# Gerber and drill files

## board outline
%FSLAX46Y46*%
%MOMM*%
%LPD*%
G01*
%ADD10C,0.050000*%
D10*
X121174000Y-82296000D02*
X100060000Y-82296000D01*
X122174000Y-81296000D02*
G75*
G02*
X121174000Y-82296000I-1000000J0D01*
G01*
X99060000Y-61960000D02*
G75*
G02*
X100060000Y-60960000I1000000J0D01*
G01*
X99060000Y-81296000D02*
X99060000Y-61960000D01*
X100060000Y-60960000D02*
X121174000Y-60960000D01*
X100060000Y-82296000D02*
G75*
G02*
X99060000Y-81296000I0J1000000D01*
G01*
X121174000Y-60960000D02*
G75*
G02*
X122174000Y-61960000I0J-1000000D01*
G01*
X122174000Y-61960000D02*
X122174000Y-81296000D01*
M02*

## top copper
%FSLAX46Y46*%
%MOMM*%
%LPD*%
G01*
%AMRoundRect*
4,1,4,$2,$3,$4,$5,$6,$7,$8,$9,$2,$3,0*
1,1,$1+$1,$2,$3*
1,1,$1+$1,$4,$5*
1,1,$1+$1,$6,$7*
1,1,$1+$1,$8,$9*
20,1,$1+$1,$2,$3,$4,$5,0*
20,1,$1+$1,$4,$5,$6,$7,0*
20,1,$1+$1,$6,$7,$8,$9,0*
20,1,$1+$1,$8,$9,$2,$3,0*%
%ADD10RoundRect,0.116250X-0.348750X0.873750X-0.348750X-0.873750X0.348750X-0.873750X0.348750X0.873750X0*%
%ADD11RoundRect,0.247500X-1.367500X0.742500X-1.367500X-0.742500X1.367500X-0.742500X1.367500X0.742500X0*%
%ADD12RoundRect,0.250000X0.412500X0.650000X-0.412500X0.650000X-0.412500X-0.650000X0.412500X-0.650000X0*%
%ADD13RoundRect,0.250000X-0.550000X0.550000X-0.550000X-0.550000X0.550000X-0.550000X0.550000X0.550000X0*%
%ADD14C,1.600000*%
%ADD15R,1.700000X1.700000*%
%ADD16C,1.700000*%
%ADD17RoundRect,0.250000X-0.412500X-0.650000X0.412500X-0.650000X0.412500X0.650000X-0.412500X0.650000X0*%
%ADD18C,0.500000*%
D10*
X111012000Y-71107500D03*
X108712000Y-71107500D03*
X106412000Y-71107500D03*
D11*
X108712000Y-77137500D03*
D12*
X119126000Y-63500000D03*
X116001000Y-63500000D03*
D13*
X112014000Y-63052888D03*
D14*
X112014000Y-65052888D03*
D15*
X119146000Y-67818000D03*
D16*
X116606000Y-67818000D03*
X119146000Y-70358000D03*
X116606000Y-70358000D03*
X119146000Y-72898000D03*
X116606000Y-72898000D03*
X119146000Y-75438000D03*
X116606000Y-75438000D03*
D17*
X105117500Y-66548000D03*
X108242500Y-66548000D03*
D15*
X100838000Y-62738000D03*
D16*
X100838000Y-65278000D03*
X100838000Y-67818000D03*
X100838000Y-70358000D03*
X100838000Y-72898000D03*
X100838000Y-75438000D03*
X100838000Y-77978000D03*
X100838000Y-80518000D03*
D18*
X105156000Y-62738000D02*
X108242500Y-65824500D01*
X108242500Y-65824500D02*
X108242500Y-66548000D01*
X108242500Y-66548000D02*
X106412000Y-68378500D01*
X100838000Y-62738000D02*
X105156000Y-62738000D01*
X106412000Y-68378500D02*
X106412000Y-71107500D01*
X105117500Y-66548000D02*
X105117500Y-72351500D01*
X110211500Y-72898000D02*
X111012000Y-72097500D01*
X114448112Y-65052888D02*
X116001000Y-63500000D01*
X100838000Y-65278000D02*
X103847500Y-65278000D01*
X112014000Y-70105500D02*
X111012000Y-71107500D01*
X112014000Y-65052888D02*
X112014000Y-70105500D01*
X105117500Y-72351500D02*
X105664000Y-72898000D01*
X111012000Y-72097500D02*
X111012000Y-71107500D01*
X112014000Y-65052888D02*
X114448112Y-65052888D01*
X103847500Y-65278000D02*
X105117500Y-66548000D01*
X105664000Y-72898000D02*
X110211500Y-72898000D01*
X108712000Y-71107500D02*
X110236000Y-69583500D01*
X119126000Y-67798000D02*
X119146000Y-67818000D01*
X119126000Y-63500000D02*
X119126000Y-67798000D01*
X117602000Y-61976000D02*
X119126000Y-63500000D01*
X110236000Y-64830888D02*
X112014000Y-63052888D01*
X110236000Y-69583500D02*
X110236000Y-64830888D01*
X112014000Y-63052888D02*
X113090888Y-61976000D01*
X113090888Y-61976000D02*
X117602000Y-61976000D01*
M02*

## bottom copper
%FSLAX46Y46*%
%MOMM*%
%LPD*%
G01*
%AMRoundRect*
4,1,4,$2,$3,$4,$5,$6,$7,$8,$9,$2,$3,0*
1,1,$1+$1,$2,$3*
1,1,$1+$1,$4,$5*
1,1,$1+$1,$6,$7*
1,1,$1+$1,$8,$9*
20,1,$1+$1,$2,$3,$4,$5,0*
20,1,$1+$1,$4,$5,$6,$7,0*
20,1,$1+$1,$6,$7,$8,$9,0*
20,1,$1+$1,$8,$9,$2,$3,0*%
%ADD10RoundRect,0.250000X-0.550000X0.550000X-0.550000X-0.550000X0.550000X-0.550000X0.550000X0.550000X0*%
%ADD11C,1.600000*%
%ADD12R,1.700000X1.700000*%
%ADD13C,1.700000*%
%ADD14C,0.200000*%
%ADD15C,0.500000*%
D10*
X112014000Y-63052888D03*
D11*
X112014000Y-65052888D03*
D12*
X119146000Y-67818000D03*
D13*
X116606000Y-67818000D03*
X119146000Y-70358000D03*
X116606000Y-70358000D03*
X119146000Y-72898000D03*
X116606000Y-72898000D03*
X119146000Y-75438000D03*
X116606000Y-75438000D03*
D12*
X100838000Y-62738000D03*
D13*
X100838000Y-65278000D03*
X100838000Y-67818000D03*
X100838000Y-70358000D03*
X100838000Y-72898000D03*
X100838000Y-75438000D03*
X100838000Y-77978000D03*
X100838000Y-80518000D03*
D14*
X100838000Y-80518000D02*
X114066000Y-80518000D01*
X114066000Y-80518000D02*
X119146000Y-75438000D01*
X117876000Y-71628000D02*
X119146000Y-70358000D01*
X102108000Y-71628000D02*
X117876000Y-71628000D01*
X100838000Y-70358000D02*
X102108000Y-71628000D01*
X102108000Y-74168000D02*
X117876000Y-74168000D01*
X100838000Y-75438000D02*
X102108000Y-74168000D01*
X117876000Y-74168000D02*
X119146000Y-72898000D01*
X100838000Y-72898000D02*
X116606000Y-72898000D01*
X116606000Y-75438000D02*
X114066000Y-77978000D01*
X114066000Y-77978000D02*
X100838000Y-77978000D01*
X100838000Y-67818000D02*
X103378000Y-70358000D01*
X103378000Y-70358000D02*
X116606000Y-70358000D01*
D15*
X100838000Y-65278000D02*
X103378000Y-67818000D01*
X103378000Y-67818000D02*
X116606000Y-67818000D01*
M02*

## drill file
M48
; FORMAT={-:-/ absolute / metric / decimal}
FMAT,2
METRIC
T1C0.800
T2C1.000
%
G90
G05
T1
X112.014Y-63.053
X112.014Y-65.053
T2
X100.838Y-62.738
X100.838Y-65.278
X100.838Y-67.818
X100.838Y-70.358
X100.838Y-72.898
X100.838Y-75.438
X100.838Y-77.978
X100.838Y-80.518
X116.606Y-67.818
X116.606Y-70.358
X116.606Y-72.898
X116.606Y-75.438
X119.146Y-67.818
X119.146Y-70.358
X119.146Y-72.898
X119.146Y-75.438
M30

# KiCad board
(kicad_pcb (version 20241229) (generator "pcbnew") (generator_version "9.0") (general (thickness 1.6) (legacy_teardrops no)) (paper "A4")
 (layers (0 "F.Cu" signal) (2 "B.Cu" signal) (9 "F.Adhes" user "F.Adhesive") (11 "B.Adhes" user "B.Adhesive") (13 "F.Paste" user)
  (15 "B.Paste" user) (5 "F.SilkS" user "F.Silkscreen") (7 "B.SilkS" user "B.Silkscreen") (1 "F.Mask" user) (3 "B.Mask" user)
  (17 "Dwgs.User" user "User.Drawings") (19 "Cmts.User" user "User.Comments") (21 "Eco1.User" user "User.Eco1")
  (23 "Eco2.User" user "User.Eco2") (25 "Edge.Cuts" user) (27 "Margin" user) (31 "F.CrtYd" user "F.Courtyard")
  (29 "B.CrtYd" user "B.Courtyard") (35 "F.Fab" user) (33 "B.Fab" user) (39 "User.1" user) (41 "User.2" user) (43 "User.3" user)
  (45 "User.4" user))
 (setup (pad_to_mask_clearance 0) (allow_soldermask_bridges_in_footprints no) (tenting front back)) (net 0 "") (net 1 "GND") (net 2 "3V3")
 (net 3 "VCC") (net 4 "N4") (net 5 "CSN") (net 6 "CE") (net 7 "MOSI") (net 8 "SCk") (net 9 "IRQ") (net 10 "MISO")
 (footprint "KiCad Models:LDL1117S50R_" (layer "F.Cu") (at 108.712 74.1225 -90)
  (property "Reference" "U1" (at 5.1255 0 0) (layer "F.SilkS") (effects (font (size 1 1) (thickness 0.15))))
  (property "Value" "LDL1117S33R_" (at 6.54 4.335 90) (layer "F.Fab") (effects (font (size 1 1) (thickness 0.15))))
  (pad "1" smd roundrect (at -3.015 -2.3 270) (size 1.98 0.93) (layers "F.Cu" "F.Mask" "F.Paste") (roundrect_rratio 0.125) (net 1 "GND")
   (solder_mask_margin 0.102))
  (pad "2" smd roundrect (at -3.015 0 270) (size 1.98 0.93) (layers "F.Cu" "F.Mask" "F.Paste") (roundrect_rratio 0.125) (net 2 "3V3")
   (solder_mask_margin 0.102))
  (pad "3" smd roundrect (at -3.015 2.3 270) (size 1.98 0.93) (layers "F.Cu" "F.Mask" "F.Paste") (roundrect_rratio 0.125) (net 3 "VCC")
   (solder_mask_margin 0.102))
  (pad "4" smd roundrect (at 3.015 0 270) (size 1.98 3.23) (layers "F.Cu" "F.Mask" "F.Paste") (roundrect_rratio 0.125) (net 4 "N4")
   (solder_mask_margin 0.102)))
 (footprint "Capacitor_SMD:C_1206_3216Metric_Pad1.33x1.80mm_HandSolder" (layer "F.Cu") (at 117.5635 63.5 180)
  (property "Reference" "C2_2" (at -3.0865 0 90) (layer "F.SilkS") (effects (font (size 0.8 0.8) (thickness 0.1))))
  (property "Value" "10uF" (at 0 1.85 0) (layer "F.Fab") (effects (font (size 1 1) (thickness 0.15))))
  (pad "1" smd roundrect (at -1.5625 0 180) (size 1.325 1.8) (layers "F.Cu" "F.Mask" "F.Paste") (roundrect_rratio 0.188679) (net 2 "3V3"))
  (pad "2" smd roundrect (at 1.5625 0 180) (size 1.325 1.8) (layers "F.Cu" "F.Mask" "F.Paste") (roundrect_rratio 0.188679) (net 1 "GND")))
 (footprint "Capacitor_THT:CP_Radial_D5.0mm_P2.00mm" (layer "F.Cu") (at 112.014 63.052888 -90)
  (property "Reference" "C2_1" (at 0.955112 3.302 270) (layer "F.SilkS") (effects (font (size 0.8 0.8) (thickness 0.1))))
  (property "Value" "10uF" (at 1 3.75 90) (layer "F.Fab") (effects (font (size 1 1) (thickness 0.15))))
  (pad "1" thru_hole roundrect (at 0 0 270) (size 1.6 1.6) (drill 0.8) (layers "*.Cu" "*.Mask") (remove_unused_layers no)
   (roundrect_rratio 0.15625) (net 2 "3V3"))
  (pad "2" thru_hole circle (at 2 0 270) (size 1.6 1.6) (drill 0.8) (layers "*.Cu" "*.Mask") (remove_unused_layers no) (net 1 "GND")))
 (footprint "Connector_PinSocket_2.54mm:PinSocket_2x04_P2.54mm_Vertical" (layer "F.Cu") (at 119.146 67.818)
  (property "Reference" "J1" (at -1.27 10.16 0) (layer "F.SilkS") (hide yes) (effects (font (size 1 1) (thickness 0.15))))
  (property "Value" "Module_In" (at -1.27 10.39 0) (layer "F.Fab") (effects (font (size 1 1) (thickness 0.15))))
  (pad "1" thru_hole rect (at 0 0) (size 1.7 1.7) (drill 1) (layers "*.Cu" "*.Mask") (remove_unused_layers no) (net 2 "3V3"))
  (pad "2" thru_hole circle (at -2.54 0) (size 1.7 1.7) (drill 1) (layers "*.Cu" "*.Mask") (remove_unused_layers no) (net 1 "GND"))
  (pad "3" thru_hole circle (at 0 2.54) (size 1.7 1.7) (drill 1) (layers "*.Cu" "*.Mask") (remove_unused_layers no) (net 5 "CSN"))
  (pad "4" thru_hole circle (at -2.54 2.54) (size 1.7 1.7) (drill 1) (layers "*.Cu" "*.Mask") (remove_unused_layers no) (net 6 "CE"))
  (pad "5" thru_hole circle (at 0 5.08) (size 1.7 1.7) (drill 1) (layers "*.Cu" "*.Mask") (remove_unused_layers no) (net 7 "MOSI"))
  (pad "6" thru_hole circle (at -2.54 5.08) (size 1.7 1.7) (drill 1) (layers "*.Cu" "*.Mask") (remove_unused_layers no) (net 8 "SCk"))
  (pad "7" thru_hole circle (at 0 7.62) (size 1.7 1.7) (drill 1) (layers "*.Cu" "*.Mask") (remove_unused_layers no) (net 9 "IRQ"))
  (pad "8" thru_hole circle (at -2.54 7.62) (size 1.7 1.7) (drill 1) (layers "*.Cu" "*.Mask") (remove_unused_layers no) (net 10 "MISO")))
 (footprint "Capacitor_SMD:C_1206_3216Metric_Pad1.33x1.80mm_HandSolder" (layer "F.Cu") (at 106.68 66.548)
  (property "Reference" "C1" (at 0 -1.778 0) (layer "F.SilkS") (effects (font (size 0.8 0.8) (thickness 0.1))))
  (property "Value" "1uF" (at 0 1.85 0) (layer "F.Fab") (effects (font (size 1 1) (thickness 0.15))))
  (pad "1" smd roundrect (at -1.5625 0) (size 1.325 1.8) (layers "F.Cu" "F.Mask" "F.Paste") (roundrect_rratio 0.188679) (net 1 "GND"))
  (pad "2" smd roundrect (at 1.5625 0) (size 1.325 1.8) (layers "F.Cu" "F.Mask" "F.Paste") (roundrect_rratio 0.188679) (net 3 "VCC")))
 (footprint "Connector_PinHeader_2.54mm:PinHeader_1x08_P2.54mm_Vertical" (layer "B.Cu") (at 100.838 62.738 180)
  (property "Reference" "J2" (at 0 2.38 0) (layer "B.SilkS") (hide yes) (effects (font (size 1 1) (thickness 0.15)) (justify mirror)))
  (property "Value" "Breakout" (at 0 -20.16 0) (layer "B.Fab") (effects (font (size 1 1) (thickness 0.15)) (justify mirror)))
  (pad "1" thru_hole rect (at 0 0 180) (size 1.7 1.7) (drill 1) (layers "*.Cu" "*.Mask") (remove_unused_layers no) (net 3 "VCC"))
  (pad "2" thru_hole circle (at 0 -2.54 180) (size 1.7 1.7) (drill 1) (layers "*.Cu" "*.Mask") (remove_unused_layers no) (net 1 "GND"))
  (pad "3" thru_hole circle (at 0 -5.08 180) (size 1.7 1.7) (drill 1) (layers "*.Cu" "*.Mask") (remove_unused_layers no) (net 6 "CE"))
  (pad "4" thru_hole circle (at 0 -7.62 180) (size 1.7 1.7) (drill 1) (layers "*.Cu" "*.Mask") (remove_unused_layers no) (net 5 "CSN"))
  (pad "5" thru_hole circle (at 0 -10.16 180) (size 1.7 1.7) (drill 1) (layers "*.Cu" "*.Mask") (remove_unused_layers no) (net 8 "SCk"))
  (pad "6" thru_hole circle (at 0 -12.7 180) (size 1.7 1.7) (drill 1) (layers "*.Cu" "*.Mask") (remove_unused_layers no) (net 7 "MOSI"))
  (pad "7" thru_hole circle (at 0 -15.24 180) (size 1.7 1.7) (drill 1) (layers "*.Cu" "*.Mask") (remove_unused_layers no) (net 10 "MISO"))
  (pad "8" thru_hole circle (at 0 -17.78 180) (size 1.7 1.7) (drill 1) (layers "*.Cu" "*.Mask") (remove_unused_layers no) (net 9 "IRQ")))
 (gr_line (start 121.174 82.296) (end 100.06 82.296) (stroke (width 0.05) (type default)) (layer "Edge.Cuts"))
 (gr_arc (start 122.174 81.296) (mid 121.881107 82.003107) (end 121.174 82.296) (stroke (width 0.05) (type default)) (layer "Edge.Cuts"))
 (gr_arc (start 99.06 61.96) (mid 99.352893 61.252893) (end 100.06 60.96) (stroke (width 0.05) (type default)) (layer "Edge.Cuts"))
 (gr_line (start 99.06 81.296) (end 99.06 61.96) (stroke (width 0.05) (type default)) (layer "Edge.Cuts"))
 (gr_line (start 100.06 60.96) (end 121.174 60.96) (stroke (width 0.05) (type default)) (layer "Edge.Cuts"))
 (gr_arc (start 100.06 82.296) (mid 99.352893 82.003107) (end 99.06 81.296) (stroke (width 0.05) (type default)) (layer "Edge.Cuts"))
 (gr_arc (start 121.174 60.96) (mid 121.881107 61.252893) (end 122.174 61.96) (stroke (width 0.05) (type default)) (layer "Edge.Cuts"))
 (gr_line (start 122.174 61.96) (end 122.174 81.296) (stroke (width 0.05) (type default)) (layer "Edge.Cuts"))
 (segment (start 100.838 80.518) (end 114.066 80.518) (width 0.2) (layer "B.Cu") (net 9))
 (segment (start 114.066 80.518) (end 119.146 75.438) (width 0.2) (layer "B.Cu") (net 9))
 (segment (start 117.876 71.628) (end 119.146 70.358) (width 0.2) (layer "B.Cu") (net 5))
 (segment (start 102.108 71.628) (end 117.876 71.628) (width 0.2) (layer "B.Cu") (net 5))
 (segment (start 100.838 70.358) (end 102.108 71.628) (width 0.2) (layer "B.Cu") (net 5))
 (segment (start 102.108 74.168) (end 117.876 74.168) (width 0.2) (layer "B.Cu") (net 7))
 (segment (start 100.838 75.438) (end 102.108 74.168) (width 0.2) (layer "B.Cu") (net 7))
 (segment (start 117.876 74.168) (end 119.146 72.898) (width 0.2) (layer "B.Cu") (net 7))
 (segment (start 100.838 72.898) (end 116.606 72.898) (width 0.2) (layer "B.Cu") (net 8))
 (segment (start 116.606 75.438) (end 114.066 77.978) (width 0.2) (layer "B.Cu") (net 10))
 (segment (start 114.066 77.978) (end 100.838 77.978) (width 0.2) (layer "B.Cu") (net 10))
 (segment (start 105.156 62.738) (end 108.2425 65.8245) (width 0.5) (layer "F.Cu") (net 3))
 (segment (start 108.2425 65.8245) (end 108.2425 66.548) (width 0.5) (layer "F.Cu") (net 3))
 (segment (start 108.2425 66.548) (end 106.412 68.3785) (width 0.5) (layer "F.Cu") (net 3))
 (segment (start 100.838 62.738) (end 105.156 62.738) (width 0.5) (layer "F.Cu") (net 3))
 (segment (start 106.412 68.3785) (end 106.412 71.1075) (width 0.5) (layer "F.Cu") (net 3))
 (segment (start 100.838 67.818) (end 103.378 70.358) (width 0.2) (layer "B.Cu") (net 6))
 (segment (start 103.378 70.358) (end 116.606 70.358) (width 0.2) (layer "B.Cu") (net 6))
 (segment (start 105.1175 66.548) (end 105.1175 72.3515) (width 0.5) (layer "F.Cu") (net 1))
 (segment (start 110.2115 72.898) (end 111.012 72.0975) (width 0.5) (layer "F.Cu") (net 1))
 (segment (start 114.448112 65.052888) (end 116.001 63.5) (width 0.5) (layer "F.Cu") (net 1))
 (segment (start 100.838 65.278) (end 103.8475 65.278) (width 0.5) (layer "F.Cu") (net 1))
 (segment (start 112.014 70.1055) (end 111.012 71.1075) (width 0.5) (layer "F.Cu") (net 1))
 (segment (start 112.014 65.052888) (end 112.014 70.1055) (width 0.5) (layer "F.Cu") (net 1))
 (segment (start 105.1175 72.3515) (end 105.664 72.898) (width 0.5) (layer "F.Cu") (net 1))
 (segment (start 111.012 72.0975) (end 111.012 71.1075) (width 0.5) (layer "F.Cu") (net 1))
 (segment (start 112.014 65.052888) (end 114.448112 65.052888) (width 0.5) (layer "F.Cu") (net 1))
 (segment (start 103.8475 65.278) (end 105.1175 66.548) (width 0.5) (layer "F.Cu") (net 1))
 (segment (start 105.664 72.898) (end 110.2115 72.898) (width 0.5) (layer "F.Cu") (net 1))
 (segment (start 100.838 65.278) (end 103.378 67.818) (width 0.5) (layer "B.Cu") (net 1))
 (segment (start 103.378 67.818) (end 116.606 67.818) (width 0.5) (layer "B.Cu") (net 1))
 (segment (start 108.712 71.1075) (end 110.236 69.5835) (width 0.5) (layer "F.Cu") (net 2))
 (segment (start 119.126 67.798) (end 119.146 67.818) (width 0.5) (layer "F.Cu") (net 2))
 (segment (start 119.126 63.5) (end 119.126 67.798) (width 0.5) (layer "F.Cu") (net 2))
 (segment (start 117.602 61.976) (end 119.126 63.5) (width 0.5) (layer "F.Cu") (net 2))
 (segment (start 110.236 64.830888) (end 112.014 63.052888) (width 0.5) (layer "F.Cu") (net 2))
 (segment (start 110.236 69.5835) (end 110.236 64.830888) (width 0.5) (layer "F.Cu") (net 2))
 (segment (start 112.014 63.052888) (end 113.090888 61.976) (width 0.5) (layer "F.Cu") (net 2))
 (segment (start 113.090888 61.976) (end 117.602 61.976) (width 0.5) (layer "F.Cu") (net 2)))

